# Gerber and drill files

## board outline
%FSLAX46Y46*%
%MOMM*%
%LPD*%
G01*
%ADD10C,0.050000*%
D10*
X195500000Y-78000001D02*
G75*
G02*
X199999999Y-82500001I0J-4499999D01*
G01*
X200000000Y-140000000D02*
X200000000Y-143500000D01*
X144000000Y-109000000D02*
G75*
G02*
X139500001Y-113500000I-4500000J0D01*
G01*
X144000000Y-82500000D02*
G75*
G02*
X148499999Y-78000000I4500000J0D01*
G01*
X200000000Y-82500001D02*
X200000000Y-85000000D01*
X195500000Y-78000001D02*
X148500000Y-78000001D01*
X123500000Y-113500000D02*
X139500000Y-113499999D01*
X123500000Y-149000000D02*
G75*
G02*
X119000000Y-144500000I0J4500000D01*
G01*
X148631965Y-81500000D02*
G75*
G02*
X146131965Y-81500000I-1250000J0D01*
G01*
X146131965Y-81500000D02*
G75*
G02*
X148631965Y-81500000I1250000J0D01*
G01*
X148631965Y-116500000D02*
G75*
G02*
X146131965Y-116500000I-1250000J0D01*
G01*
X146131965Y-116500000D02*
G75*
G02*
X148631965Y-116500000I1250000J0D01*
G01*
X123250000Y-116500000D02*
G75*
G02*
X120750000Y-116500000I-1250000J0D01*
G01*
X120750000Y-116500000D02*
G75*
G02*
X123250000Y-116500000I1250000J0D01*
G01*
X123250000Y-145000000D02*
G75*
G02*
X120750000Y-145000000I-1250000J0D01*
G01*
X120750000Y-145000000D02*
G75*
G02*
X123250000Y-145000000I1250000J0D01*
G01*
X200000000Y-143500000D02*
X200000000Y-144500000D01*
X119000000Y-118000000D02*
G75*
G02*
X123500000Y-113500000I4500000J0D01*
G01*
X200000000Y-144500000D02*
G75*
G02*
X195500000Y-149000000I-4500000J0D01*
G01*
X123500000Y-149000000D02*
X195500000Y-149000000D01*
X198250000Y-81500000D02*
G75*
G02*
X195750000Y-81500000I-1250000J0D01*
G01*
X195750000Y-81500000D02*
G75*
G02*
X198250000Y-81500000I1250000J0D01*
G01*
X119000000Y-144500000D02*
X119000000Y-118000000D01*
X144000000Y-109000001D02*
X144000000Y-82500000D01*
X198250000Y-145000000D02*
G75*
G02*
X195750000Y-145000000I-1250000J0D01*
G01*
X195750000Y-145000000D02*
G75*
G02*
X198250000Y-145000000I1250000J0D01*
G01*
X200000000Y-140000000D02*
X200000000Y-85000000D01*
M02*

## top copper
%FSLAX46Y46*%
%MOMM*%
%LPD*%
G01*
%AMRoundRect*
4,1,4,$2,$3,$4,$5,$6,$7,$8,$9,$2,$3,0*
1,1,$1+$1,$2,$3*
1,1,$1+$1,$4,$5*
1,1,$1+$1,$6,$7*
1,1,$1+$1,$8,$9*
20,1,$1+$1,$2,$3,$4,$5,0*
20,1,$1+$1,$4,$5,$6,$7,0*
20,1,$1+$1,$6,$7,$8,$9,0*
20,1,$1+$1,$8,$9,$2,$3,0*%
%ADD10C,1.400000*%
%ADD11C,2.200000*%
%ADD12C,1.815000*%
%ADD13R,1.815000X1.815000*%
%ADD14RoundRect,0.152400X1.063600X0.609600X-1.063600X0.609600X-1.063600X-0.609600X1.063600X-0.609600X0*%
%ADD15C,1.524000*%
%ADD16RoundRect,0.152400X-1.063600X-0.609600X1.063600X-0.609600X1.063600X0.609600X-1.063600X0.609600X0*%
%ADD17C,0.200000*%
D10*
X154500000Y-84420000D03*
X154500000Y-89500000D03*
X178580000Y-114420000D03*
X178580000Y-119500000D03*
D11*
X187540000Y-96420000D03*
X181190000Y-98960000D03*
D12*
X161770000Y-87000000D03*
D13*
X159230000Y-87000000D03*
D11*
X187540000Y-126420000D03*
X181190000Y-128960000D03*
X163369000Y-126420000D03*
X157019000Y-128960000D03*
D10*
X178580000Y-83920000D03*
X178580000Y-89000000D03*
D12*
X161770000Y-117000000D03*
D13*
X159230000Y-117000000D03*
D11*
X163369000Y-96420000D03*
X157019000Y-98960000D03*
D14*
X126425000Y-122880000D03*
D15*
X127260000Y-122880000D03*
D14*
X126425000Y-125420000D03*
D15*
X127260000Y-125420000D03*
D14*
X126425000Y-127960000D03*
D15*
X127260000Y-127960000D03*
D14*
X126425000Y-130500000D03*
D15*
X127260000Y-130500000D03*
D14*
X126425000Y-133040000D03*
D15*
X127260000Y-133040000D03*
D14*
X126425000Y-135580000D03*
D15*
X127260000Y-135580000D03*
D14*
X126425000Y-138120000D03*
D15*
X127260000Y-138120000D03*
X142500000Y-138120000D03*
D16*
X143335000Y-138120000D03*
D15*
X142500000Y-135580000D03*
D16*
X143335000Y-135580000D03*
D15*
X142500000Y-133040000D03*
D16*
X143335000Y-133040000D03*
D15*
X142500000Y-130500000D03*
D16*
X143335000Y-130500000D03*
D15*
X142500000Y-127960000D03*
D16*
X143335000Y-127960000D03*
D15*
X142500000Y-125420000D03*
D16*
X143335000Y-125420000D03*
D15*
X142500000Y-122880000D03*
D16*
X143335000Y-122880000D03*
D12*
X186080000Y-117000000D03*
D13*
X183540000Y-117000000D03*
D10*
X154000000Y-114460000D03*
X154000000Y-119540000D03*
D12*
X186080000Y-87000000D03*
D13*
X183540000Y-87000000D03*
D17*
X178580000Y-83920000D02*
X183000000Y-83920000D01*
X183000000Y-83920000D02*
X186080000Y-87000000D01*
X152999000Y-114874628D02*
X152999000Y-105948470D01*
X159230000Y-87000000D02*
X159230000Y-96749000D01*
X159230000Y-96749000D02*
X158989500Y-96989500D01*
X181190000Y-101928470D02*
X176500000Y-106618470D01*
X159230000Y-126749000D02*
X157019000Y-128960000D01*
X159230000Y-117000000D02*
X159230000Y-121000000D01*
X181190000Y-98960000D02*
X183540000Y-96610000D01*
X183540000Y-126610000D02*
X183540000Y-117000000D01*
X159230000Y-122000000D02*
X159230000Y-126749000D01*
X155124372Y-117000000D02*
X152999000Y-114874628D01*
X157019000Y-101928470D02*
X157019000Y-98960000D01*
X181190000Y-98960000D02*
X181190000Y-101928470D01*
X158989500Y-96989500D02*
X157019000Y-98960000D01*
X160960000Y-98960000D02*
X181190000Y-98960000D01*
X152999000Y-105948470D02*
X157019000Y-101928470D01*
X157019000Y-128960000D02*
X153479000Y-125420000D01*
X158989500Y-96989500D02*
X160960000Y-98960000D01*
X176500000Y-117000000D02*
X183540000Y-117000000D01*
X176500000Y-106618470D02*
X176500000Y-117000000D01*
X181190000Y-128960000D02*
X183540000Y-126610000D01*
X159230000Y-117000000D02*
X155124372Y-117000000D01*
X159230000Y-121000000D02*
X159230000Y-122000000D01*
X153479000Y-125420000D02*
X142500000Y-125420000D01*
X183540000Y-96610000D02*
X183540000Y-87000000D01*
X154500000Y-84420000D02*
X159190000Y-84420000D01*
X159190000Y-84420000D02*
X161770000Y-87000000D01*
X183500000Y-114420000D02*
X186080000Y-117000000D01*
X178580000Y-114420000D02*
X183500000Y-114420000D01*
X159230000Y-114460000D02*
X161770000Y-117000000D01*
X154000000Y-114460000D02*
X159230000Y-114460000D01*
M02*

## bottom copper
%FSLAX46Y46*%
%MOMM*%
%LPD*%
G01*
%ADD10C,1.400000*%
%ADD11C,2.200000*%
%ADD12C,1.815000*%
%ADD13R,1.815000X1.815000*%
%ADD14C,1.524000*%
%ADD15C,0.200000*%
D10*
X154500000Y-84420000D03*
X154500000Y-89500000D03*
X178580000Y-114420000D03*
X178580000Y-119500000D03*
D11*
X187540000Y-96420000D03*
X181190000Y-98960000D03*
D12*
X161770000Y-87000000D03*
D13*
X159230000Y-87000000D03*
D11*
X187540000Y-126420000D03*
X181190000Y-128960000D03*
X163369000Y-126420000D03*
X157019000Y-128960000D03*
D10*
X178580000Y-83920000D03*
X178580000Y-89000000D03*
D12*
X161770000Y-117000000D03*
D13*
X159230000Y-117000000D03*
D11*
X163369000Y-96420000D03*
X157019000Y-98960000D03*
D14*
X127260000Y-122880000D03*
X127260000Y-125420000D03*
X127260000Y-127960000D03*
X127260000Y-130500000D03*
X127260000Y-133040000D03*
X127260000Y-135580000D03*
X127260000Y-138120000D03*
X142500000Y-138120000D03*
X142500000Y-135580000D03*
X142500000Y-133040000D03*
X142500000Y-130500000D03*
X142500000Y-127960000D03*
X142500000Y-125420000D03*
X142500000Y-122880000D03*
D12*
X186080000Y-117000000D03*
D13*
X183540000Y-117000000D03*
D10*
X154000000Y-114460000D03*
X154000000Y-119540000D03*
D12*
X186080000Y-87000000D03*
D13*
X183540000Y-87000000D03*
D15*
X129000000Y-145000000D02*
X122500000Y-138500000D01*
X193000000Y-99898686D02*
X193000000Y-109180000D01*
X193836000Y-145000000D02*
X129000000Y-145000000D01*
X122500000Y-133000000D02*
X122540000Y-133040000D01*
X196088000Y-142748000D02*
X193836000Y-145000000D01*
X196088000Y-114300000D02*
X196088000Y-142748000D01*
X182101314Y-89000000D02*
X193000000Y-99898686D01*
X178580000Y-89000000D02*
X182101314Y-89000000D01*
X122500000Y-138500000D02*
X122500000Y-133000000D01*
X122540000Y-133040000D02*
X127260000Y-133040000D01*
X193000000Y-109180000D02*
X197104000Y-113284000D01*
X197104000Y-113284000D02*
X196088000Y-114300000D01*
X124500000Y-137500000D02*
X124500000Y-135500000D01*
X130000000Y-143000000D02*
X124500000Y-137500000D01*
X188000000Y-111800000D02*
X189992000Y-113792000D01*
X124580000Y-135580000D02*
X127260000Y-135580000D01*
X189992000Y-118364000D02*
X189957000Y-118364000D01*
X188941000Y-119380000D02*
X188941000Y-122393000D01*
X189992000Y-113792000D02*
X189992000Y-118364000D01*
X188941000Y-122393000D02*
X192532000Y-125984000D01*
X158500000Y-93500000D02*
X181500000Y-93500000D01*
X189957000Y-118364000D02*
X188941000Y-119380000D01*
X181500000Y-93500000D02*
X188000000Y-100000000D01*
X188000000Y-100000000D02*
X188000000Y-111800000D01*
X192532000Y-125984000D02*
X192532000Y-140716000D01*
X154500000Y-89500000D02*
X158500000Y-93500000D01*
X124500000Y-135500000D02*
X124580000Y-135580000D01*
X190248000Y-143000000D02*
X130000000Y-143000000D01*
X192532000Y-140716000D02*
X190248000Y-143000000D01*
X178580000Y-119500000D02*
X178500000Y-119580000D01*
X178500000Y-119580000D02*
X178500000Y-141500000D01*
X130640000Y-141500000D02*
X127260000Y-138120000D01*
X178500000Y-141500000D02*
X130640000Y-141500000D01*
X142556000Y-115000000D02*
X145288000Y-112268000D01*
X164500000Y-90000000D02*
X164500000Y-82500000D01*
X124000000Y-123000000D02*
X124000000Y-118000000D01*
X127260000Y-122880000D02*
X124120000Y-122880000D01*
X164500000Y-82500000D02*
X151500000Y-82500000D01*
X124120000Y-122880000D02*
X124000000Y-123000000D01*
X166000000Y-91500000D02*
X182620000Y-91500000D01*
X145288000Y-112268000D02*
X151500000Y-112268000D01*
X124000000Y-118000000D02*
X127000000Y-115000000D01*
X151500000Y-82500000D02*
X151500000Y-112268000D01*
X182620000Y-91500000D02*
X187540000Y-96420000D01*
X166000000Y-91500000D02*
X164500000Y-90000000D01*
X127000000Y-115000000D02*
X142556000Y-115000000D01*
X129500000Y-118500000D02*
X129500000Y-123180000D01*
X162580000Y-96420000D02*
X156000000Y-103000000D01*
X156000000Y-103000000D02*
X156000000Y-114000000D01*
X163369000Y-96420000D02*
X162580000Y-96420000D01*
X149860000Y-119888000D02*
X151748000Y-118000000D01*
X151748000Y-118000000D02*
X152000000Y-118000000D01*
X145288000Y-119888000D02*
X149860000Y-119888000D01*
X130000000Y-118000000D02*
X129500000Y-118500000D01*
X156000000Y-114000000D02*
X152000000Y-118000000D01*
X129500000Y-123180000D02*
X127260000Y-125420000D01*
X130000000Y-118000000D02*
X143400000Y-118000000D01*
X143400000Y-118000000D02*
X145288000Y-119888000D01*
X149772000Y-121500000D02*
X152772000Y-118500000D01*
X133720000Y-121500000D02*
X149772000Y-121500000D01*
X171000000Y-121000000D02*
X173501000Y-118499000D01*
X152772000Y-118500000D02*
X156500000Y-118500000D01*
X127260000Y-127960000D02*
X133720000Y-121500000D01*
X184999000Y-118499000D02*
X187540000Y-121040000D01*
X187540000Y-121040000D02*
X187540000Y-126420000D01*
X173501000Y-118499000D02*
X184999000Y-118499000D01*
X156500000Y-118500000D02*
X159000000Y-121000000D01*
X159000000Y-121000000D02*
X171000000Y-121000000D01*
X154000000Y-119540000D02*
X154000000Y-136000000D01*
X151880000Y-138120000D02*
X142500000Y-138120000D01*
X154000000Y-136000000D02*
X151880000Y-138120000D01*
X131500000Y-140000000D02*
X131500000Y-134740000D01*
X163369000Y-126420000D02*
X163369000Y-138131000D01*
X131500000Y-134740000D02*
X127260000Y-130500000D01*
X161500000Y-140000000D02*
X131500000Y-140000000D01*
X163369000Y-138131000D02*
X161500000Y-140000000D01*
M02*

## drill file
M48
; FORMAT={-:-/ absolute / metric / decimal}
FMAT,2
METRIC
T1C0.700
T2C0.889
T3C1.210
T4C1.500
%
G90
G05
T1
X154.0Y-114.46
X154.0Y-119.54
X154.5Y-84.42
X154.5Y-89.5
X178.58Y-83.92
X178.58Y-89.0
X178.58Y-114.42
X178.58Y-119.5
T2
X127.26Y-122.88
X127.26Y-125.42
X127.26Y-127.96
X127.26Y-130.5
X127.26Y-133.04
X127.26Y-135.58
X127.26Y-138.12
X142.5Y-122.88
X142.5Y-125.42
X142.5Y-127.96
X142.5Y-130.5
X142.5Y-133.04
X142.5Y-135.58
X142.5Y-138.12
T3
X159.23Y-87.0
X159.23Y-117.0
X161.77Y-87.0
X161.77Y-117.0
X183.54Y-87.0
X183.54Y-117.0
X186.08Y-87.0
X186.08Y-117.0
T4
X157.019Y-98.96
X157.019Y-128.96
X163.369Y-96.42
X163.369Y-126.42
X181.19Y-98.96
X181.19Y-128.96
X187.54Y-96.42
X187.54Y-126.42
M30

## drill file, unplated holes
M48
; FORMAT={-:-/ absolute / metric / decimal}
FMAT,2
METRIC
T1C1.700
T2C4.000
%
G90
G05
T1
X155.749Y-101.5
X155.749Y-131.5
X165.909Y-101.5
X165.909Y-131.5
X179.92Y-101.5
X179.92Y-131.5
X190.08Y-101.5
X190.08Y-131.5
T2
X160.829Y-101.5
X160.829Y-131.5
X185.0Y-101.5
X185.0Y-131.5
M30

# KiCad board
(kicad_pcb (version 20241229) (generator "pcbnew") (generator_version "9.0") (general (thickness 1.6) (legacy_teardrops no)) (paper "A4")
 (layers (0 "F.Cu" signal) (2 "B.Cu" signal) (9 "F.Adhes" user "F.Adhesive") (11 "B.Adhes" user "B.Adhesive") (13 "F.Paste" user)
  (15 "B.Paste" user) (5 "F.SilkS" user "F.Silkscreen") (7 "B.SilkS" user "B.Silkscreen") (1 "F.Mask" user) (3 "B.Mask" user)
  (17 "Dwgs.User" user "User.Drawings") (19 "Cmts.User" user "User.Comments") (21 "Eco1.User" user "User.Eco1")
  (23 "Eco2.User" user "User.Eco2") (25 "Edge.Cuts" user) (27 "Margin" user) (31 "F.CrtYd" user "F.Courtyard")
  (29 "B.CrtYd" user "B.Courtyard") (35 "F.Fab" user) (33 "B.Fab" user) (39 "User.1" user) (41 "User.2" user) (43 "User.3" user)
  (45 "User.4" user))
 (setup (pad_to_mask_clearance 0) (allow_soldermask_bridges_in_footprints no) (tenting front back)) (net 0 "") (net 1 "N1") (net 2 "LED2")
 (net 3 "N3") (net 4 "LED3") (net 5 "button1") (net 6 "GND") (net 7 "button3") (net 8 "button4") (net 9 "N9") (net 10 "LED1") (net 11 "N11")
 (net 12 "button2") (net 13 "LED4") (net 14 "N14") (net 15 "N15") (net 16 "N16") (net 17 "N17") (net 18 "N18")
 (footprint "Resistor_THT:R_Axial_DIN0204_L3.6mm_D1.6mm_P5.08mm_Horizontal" (layer "F.Cu") (at 154.5 84.42 -90)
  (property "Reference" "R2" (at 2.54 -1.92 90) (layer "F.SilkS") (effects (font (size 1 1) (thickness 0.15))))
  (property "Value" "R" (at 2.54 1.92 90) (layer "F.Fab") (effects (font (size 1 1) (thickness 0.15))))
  (pad "1" thru_hole circle (at 0 0 270) (size 1.4 1.4) (drill 0.7) (layers "*.Cu" "*.Mask") (remove_unused_layers no) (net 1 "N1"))
  (pad "2" thru_hole circle (at 5.08 0 270) (size 1.4 1.4) (drill 0.7) (layers "*.Cu" "*.Mask") (remove_unused_layers no) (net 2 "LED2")))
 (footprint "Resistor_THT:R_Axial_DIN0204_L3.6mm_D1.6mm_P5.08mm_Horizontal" (layer "F.Cu") (at 178.58 114.42 -90)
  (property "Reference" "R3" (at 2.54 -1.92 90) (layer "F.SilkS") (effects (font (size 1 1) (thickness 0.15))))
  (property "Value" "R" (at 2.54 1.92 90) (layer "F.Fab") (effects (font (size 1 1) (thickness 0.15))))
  (pad "1" thru_hole circle (at 0 0 270) (size 1.4 1.4) (drill 0.7) (layers "*.Cu" "*.Mask") (remove_unused_layers no) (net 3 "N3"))
  (pad "2" thru_hole circle (at 5.08 0 270) (size 1.4 1.4) (drill 0.7) (layers "*.Cu" "*.Mask") (remove_unused_layers no) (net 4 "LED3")))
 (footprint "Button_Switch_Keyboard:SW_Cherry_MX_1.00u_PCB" (layer "F.Cu") (at 187.54 96.42)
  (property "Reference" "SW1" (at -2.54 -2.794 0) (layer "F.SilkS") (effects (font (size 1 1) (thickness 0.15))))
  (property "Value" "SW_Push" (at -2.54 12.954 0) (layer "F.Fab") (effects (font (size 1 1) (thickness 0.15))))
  (pad "" np_thru_hole circle (at -7.62 5.08) (size 1.7 1.7) (drill 1.7) (layers "*.Cu" "*.Mask"))
  (pad "" np_thru_hole circle (at -2.54 5.08) (size 4 4) (drill 4) (layers "*.Cu" "*.Mask"))
  (pad "" np_thru_hole circle (at 2.54 5.08) (size 1.7 1.7) (drill 1.7) (layers "*.Cu" "*.Mask"))
  (pad "1" thru_hole circle (at 0 0) (size 2.2 2.2) (drill 1.5) (layers "*.Cu" "*.Mask") (remove_unused_layers no) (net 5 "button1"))
  (pad "2" thru_hole circle (at -6.35 2.54) (size 2.2 2.2) (drill 1.5) (layers "*.Cu" "*.Mask") (remove_unused_layers no) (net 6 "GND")))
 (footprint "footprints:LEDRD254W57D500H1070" (layer "F.Cu") (at 160.5 87)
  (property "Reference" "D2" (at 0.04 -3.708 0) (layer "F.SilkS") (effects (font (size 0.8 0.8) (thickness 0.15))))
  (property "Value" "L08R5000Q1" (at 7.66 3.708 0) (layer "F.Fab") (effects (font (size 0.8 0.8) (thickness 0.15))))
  (pad "A" thru_hole circle (at 1.27 0) (size 1.815 1.815) (drill 1.21) (layers "*.Cu" "*.Mask") (remove_unused_layers no) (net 1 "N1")
   (solder_mask_margin 0.102))
  (pad "C" thru_hole rect (at -1.27 0) (size 1.815 1.815) (drill 1.21) (layers "*.Cu" "*.Mask") (remove_unused_layers no) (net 6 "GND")
   (solder_mask_margin 0.102)))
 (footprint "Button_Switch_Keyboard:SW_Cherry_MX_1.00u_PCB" (layer "F.Cu") (at 187.54 126.42)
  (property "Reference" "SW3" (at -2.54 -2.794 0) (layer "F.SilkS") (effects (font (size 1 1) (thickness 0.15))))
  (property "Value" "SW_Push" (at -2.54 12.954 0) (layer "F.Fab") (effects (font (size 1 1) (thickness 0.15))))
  (pad "" np_thru_hole circle (at -7.62 5.08) (size 1.7 1.7) (drill 1.7) (layers "*.Cu" "*.Mask"))
  (pad "" np_thru_hole circle (at -2.54 5.08) (size 4 4) (drill 4) (layers "*.Cu" "*.Mask"))
  (pad "" np_thru_hole circle (at 2.54 5.08) (size 1.7 1.7) (drill 1.7) (layers "*.Cu" "*.Mask"))
  (pad "1" thru_hole circle (at 0 0) (size 2.2 2.2) (drill 1.5) (layers "*.Cu" "*.Mask") (remove_unused_layers no) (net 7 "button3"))
  (pad "2" thru_hole circle (at -6.35 2.54) (size 2.2 2.2) (drill 1.5) (layers "*.Cu" "*.Mask") (remove_unused_layers no) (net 6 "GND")))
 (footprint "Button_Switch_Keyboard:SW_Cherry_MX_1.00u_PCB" (layer "F.Cu") (at 163.369 126.42)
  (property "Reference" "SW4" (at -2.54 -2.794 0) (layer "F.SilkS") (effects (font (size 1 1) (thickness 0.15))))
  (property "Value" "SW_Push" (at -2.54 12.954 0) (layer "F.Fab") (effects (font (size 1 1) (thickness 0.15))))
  (pad "" np_thru_hole circle (at -7.62 5.08) (size 1.7 1.7) (drill 1.7) (layers "*.Cu" "*.Mask"))
  (pad "" np_thru_hole circle (at -2.54 5.08) (size 4 4) (drill 4) (layers "*.Cu" "*.Mask"))
  (pad "" np_thru_hole circle (at 2.54 5.08) (size 1.7 1.7) (drill 1.7) (layers "*.Cu" "*.Mask"))
  (pad "1" thru_hole circle (at 0 0) (size 2.2 2.2) (drill 1.5) (layers "*.Cu" "*.Mask") (remove_unused_layers no) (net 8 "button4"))
  (pad "2" thru_hole circle (at -6.35 2.54) (size 2.2 2.2) (drill 1.5) (layers "*.Cu" "*.Mask") (remove_unused_layers no) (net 6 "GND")))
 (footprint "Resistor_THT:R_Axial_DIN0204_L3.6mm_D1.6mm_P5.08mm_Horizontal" (layer "F.Cu") (at 178.58 83.92 -90)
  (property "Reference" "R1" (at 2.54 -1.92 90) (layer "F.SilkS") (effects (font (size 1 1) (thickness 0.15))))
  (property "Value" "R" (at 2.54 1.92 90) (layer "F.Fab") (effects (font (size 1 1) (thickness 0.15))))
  (pad "1" thru_hole circle (at 0 0 270) (size 1.4 1.4) (drill 0.7) (layers "*.Cu" "*.Mask") (remove_unused_layers no) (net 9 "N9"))
  (pad "2" thru_hole circle (at 5.08 0 270) (size 1.4 1.4) (drill 0.7) (layers "*.Cu" "*.Mask") (remove_unused_layers no) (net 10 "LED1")))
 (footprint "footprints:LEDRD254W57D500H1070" (layer "F.Cu") (at 160.5 117)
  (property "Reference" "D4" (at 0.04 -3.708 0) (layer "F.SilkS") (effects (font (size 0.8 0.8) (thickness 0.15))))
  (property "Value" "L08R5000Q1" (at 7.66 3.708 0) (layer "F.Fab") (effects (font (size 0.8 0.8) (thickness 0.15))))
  (pad "A" thru_hole circle (at 1.27 0) (size 1.815 1.815) (drill 1.21) (layers "*.Cu" "*.Mask") (remove_unused_layers no) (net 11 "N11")
   (solder_mask_margin 0.102))
  (pad "C" thru_hole rect (at -1.27 0) (size 1.815 1.815) (drill 1.21) (layers "*.Cu" "*.Mask") (remove_unused_layers no) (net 6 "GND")
   (solder_mask_margin 0.102)))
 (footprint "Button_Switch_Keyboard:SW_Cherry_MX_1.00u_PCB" (layer "F.Cu") (at 163.369 96.42)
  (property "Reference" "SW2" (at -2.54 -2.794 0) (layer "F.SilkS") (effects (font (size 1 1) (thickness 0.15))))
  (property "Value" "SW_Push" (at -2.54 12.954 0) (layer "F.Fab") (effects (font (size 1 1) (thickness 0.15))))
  (pad "" np_thru_hole circle (at -7.62 5.08) (size 1.7 1.7) (drill 1.7) (layers "*.Cu" "*.Mask"))
  (pad "" np_thru_hole circle (at -2.54 5.08) (size 4 4) (drill 4) (layers "*.Cu" "*.Mask"))
  (pad "" np_thru_hole circle (at 2.54 5.08) (size 1.7 1.7) (drill 1.7) (layers "*.Cu" "*.Mask"))
  (pad "1" thru_hole circle (at 0 0) (size 2.2 2.2) (drill 1.5) (layers "*.Cu" "*.Mask") (remove_unused_layers no) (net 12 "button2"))
  (pad "2" thru_hole circle (at -6.35 2.54) (size 2.2 2.2) (drill 1.5) (layers "*.Cu" "*.Mask") (remove_unused_layers no) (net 6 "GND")))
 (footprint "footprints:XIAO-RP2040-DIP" (layer "F.Cu") (at 134.88 130.5)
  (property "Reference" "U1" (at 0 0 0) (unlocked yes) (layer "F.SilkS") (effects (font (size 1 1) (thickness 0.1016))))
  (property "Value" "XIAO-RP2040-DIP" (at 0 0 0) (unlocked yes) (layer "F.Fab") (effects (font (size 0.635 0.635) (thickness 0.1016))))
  (pad "1" smd roundrect (at -8.455 -7.62 180) (size 2.432 1.524) (layers "F.Cu" "F.Mask") (roundrect_rratio 0.1) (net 5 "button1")
   (thermal_bridge_angle 45))
  (pad "1" thru_hole circle (at -7.62 -7.62 180) (size 1.524 1.524) (drill 0.889) (layers "*.Cu" "*.Mask") (remove_unused_layers no)
   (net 5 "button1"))
  (pad "2" smd roundrect (at -8.455 -5.08 180) (size 2.432 1.524) (layers "F.Cu" "F.Mask") (roundrect_rratio 0.1) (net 12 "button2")
   (thermal_bridge_angle 45))
  (pad "2" thru_hole circle (at -7.62 -5.08 180) (size 1.524 1.524) (drill 0.889) (layers "*.Cu" "*.Mask") (remove_unused_layers no)
   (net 12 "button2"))
  (pad "3" smd roundrect (at -8.455 -2.54 180) (size 2.432 1.524) (layers "F.Cu" "F.Mask") (roundrect_rratio 0.1) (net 7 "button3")
   (thermal_bridge_angle 45))
  (pad "3" thru_hole circle (at -7.62 -2.54 180) (size 1.524 1.524) (drill 0.889) (layers "*.Cu" "*.Mask") (remove_unused_layers no)
   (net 7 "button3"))
  (pad "4" smd roundrect (at -8.455 0 180) (size 2.432 1.524) (layers "F.Cu" "F.Mask") (roundrect_rratio 0.1) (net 8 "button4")
   (thermal_bridge_angle 45))
  (pad "4" thru_hole circle (at -7.62 0 180) (size 1.524 1.524) (drill 0.889) (layers "*.Cu" "*.Mask") (remove_unused_layers no)
   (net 8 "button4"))
  (pad "5" smd roundrect (at -8.455 2.54 180) (size 2.432 1.524) (layers "F.Cu" "F.Mask") (roundrect_rratio 0.1) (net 10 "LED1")
   (thermal_bridge_angle 45))
  (pad "5" thru_hole circle (at -7.62 2.54 180) (size 1.524 1.524) (drill 0.889) (layers "*.Cu" "*.Mask") (remove_unused_layers no)
   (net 10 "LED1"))
  (pad "6" smd roundrect (at -8.455 5.08 180) (size 2.432 1.524) (layers "F.Cu" "F.Mask") (roundrect_rratio 0.1) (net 2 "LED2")
   (thermal_bridge_angle 45))
  (pad "6" thru_hole circle (at -7.62 5.08 180) (size 1.524 1.524) (drill 0.889) (layers "*.Cu" "*.Mask") (remove_unused_layers no)
   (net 2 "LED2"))
  (pad "7" smd roundrect (at -8.455 7.62 180) (size 2.432 1.524) (layers "F.Cu" "F.Mask") (roundrect_rratio 0.1) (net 4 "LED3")
   (thermal_bridge_angle 45))
  (pad "7" thru_hole circle (at -7.62 7.62 180) (size 1.524 1.524) (drill 0.889) (layers "*.Cu" "*.Mask") (remove_unused_layers no)
   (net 4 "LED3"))
  (pad "8" thru_hole circle (at 7.62 7.62) (size 1.524 1.524) (drill 0.889) (layers "*.Cu" "*.Mask") (remove_unused_layers no)
   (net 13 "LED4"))
  (pad "8" smd roundrect (at 8.455 7.62) (size 2.432 1.524) (layers "F.Cu" "F.Mask") (roundrect_rratio 0.1) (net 13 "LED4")
   (thermal_bridge_angle 45))
  (pad "9" thru_hole circle (at 7.62 5.08) (size 1.524 1.524) (drill 0.889) (layers "*.Cu" "*.Mask") (remove_unused_layers no)
   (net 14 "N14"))
  (pad "9" smd roundrect (at 8.455 5.08) (size 2.432 1.524) (layers "F.Cu" "F.Mask") (roundrect_rratio 0.1) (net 14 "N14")
   (thermal_bridge_angle 45))
  (pad "10" thru_hole circle (at 7.62 2.54) (size 1.524 1.524) (drill 0.889) (layers "*.Cu" "*.Mask") (remove_unused_layers no)
   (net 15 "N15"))
  (pad "10" smd roundrect (at 8.455 2.54) (size 2.432 1.524) (layers "F.Cu" "F.Mask") (roundrect_rratio 0.1) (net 15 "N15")
   (thermal_bridge_angle 45))
  (pad "11" thru_hole circle (at 7.62 0) (size 1.524 1.524) (drill 0.889) (layers "*.Cu" "*.Mask") (remove_unused_layers no) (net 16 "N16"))
  (pad "11" smd roundrect (at 8.455 0) (size 2.432 1.524) (layers "F.Cu" "F.Mask") (roundrect_rratio 0.1) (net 16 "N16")
   (thermal_bridge_angle 45))
  (pad "12" thru_hole circle (at 7.62 -2.54) (size 1.524 1.524) (drill 0.889) (layers "*.Cu" "*.Mask") (remove_unused_layers no)
   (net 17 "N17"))
  (pad "12" smd roundrect (at 8.455 -2.54) (size 2.432 1.524) (layers "F.Cu" "F.Mask") (roundrect_rratio 0.1) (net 17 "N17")
   (thermal_bridge_angle 45))
  (pad "13" thru_hole circle (at 7.62 -5.08) (size 1.524 1.524) (drill 0.889) (layers "*.Cu" "*.Mask") (remove_unused_layers no)
   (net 6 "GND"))
  (pad "13" smd roundrect (at 8.455 -5.08) (size 2.432 1.524) (layers "F.Cu" "F.Mask") (roundrect_rratio 0.1) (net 6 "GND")
   (thermal_bridge_angle 45))
  (pad "14" thru_hole circle (at 7.62 -7.62) (size 1.524 1.524) (drill 0.889) (layers "*.Cu" "*.Mask") (remove_unused_layers no)
   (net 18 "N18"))
  (pad "14" smd roundrect (at 8.455 -7.62) (size 2.432 1.524) (layers "F.Cu" "F.Mask") (roundrect_rratio 0.1) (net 18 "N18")
   (thermal_bridge_angle 45)))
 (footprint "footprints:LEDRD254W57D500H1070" (layer "F.Cu") (at 184.81 117)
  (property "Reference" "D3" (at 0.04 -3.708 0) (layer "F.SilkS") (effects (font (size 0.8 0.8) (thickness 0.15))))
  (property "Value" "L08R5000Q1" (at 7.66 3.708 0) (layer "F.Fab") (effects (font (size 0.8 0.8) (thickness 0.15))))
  (pad "A" thru_hole circle (at 1.27 0) (size 1.815 1.815) (drill 1.21) (layers "*.Cu" "*.Mask") (remove_unused_layers no) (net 3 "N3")
   (solder_mask_margin 0.102))
  (pad "C" thru_hole rect (at -1.27 0) (size 1.815 1.815) (drill 1.21) (layers "*.Cu" "*.Mask") (remove_unused_layers no) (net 6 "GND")
   (solder_mask_margin 0.102)))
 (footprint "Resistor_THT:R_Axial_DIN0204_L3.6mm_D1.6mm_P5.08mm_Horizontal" (layer "F.Cu") (at 154 114.46 -90)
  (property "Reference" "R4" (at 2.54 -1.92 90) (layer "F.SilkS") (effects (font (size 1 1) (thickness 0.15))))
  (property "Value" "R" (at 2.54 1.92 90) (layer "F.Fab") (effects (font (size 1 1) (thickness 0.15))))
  (pad "1" thru_hole circle (at 0 0 270) (size 1.4 1.4) (drill 0.7) (layers "*.Cu" "*.Mask") (remove_unused_layers no) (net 11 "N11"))
  (pad "2" thru_hole circle (at 5.08 0 270) (size 1.4 1.4) (drill 0.7) (layers "*.Cu" "*.Mask") (remove_unused_layers no) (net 13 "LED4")))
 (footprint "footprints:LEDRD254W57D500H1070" (layer "F.Cu") (at 184.81 87)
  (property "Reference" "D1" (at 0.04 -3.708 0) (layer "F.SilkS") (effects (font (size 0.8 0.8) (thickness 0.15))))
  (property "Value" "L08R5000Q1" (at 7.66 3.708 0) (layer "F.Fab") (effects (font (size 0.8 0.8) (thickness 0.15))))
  (pad "A" thru_hole circle (at 1.27 0) (size 1.815 1.815) (drill 1.21) (layers "*.Cu" "*.Mask") (remove_unused_layers no) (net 9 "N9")
   (solder_mask_margin 0.102))
  (pad "C" thru_hole rect (at -1.27 0) (size 1.815 1.815) (drill 1.21) (layers "*.Cu" "*.Mask") (remove_unused_layers no) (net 6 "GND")
   (solder_mask_margin 0.102)))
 (gr_arc (start 195.5 78.000001) (mid 198.681981 79.31802) (end 200 82.500001) (stroke (width 0.05) (type default)) (layer "Edge.Cuts"))
 (gr_line (start 200 140) (end 200 143.5) (stroke (width 0.05) (type default)) (layer "Edge.Cuts"))
 (gr_arc (start 144 109) (mid 142.681982 112.181986) (end 139.500001 113.499999) (stroke (width 0.05) (type default)) (layer "Edge.Cuts"))
 (gr_arc (start 144 82.5) (mid 145.31802 79.318026) (end 148.499999 78.000001) (stroke (width 0.05) (type default)) (layer "Edge.Cuts"))
 (gr_line (start 200 82.500001) (end 200 85) (stroke (width 0.05) (type default)) (layer "Edge.Cuts"))
 (gr_line (start 195.5 78.000001) (end 148.5 78.000001) (stroke (width 0.05) (type default)) (layer "Edge.Cuts"))
 (gr_line (start 123.5 113.5) (end 139.5 113.499999) (stroke (width 0.05) (type default)) (layer "Edge.Cuts"))
 (gr_arc (start 123.5 149) (mid 120.318019 147.681981) (end 119 144.5) (stroke (width 0.05) (type default)) (layer "Edge.Cuts"))
 (gr_circle (center 147.381965 81.5) (end 148.631965 81.5) (stroke (width 0.05) (type solid)) (fill no) (layer "Edge.Cuts"))
 (gr_circle (center 147.381965 116.5) (end 148.631965 116.5) (stroke (width 0.05) (type solid)) (fill no) (layer "Edge.Cuts"))
 (gr_circle (center 122 116.5) (end 123.25 116.5) (stroke (width 0.05) (type solid)) (fill no) (layer "Edge.Cuts"))
 (gr_circle (center 122 145) (end 123.25 145) (stroke (width 0.05) (type solid)) (fill no) (layer "Edge.Cuts"))
 (gr_line (start 200 143.5) (end 200 144.5) (stroke (width 0.05) (type default)) (layer "Edge.Cuts"))
 (gr_arc (start 119 118) (mid 120.31802 114.81802) (end 123.5 113.5) (stroke (width 0.05) (type default)) (layer "Edge.Cuts"))
 (gr_arc (start 200 144.5) (mid 198.681981 147.681981) (end 195.5 149) (stroke (width 0.05) (type default)) (layer "Edge.Cuts"))
 (gr_line (start 123.5 149) (end 195.5 149) (stroke (width 0.05) (type default)) (layer "Edge.Cuts"))
 (gr_circle (center 197 81.5) (end 198.25 81.5) (stroke (width 0.05) (type solid)) (fill no) (layer "Edge.Cuts"))
 (gr_line (start 119 144.5) (end 119 118) (stroke (width 0.05) (type default)) (layer "Edge.Cuts"))
 (gr_line (start 144 109.000001) (end 144 82.5) (stroke (width 0.05) (type default)) (layer "Edge.Cuts"))
 (gr_circle (center 197 145) (end 198.25 145) (stroke (width 0.05) (type solid)) (fill no) (layer "Edge.Cuts"))
 (gr_line (start 200 140) (end 200 85) (stroke (width 0.05) (type solid)) (layer "Edge.Cuts"))
 (segment (start 178.58 83.92) (end 183 83.92) (width 0.2) (layer "F.Cu") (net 9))
 (segment (start 183 83.92) (end 186.08 87) (width 0.2) (layer "F.Cu") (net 9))
 (segment (start 152.999 114.874628) (end 152.999 105.94847) (width 0.2) (layer "F.Cu") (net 6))
 (segment (start 159.23 87) (end 159.23 96.749) (width 0.2) (layer "F.Cu") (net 6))
 (segment (start 159.23 96.749) (end 158.9895 96.9895) (width 0.2) (layer "F.Cu") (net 6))
 (segment (start 181.19 101.92847) (end 176.5 106.61847) (width 0.2) (layer "F.Cu") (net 6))
 (segment (start 159.23 126.749) (end 157.019 128.96) (width 0.2) (layer "F.Cu") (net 6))
 (segment (start 159.23 117) (end 159.23 121) (width 0.2) (layer "F.Cu") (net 6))
 (segment (start 181.19 98.96) (end 183.54 96.61) (width 0.2) (layer "F.Cu") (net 6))
 (segment (start 183.54 126.61) (end 183.54 117) (width 0.2) (layer "F.Cu") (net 6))
 (segment (start 159.23 122) (end 159.23 126.749) (width 0.2) (layer "F.Cu") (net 6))
 (segment (start 155.124372 117) (end 152.999 114.874628) (width 0.2) (layer "F.Cu") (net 6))
 (segment (start 157.019 101.92847) (end 157.019 98.96) (width 0.2) (layer "F.Cu") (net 6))
 (segment (start 181.19 98.96) (end 181.19 101.92847) (width 0.2) (layer "F.Cu") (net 6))
 (segment (start 158.9895 96.9895) (end 157.019 98.96) (width 0.2) (layer "F.Cu") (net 6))
 (segment (start 160.96 98.96) (end 181.19 98.96) (width 0.2) (layer "F.Cu") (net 6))
 (segment (start 152.999 105.94847) (end 157.019 101.92847) (width 0.2) (layer "F.Cu") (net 6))
 (segment (start 157.019 128.96) (end 153.479 125.42) (width 0.2) (layer "F.Cu") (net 6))
 (segment (start 158.9895 96.9895) (end 160.96 98.96) (width 0.2) (layer "F.Cu") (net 6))
 (segment (start 176.5 117) (end 183.54 117) (width 0.2) (layer "F.Cu") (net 6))
 (segment (start 176.5 106.61847) (end 176.5 117) (width 0.2) (layer "F.Cu") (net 6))
 (segment (start 181.19 128.96) (end 183.54 126.61) (width 0.2) (layer "F.Cu") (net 6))
 (segment (start 159.23 117) (end 155.124372 117) (width 0.2) (layer "F.Cu") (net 6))
 (segment (start 159.23 121) (end 159.23 122) (width 0.2) (layer "F.Cu") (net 6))
 (segment (start 153.479 125.42) (end 142.5 125.42) (width 0.2) (layer "F.Cu") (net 6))
 (segment (start 183.54 96.61) (end 183.54 87) (width 0.2) (layer "F.Cu") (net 6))
 (segment (start 154.5 84.42) (end 159.19 84.42) (width 0.2) (layer "F.Cu") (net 1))
 (segment (start 159.19 84.42) (end 161.77 87) (width 0.2) (layer "F.Cu") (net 1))
 (segment (start 183.5 114.42) (end 186.08 117) (width 0.2) (layer "F.Cu") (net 3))
 (segment (start 178.58 114.42) (end 183.5 114.42) (width 0.2) (layer "F.Cu") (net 3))
 (segment (start 129 145) (end 122.5 138.5) (width 0.2) (layer "B.Cu") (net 10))
 (segment (start 193 99.898686) (end 193 109.18) (width 0.2) (layer "B.Cu") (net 10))
 (segment (start 193.836 145) (end 129 145) (width 0.2) (layer "B.Cu") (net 10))
 (segment (start 122.5 133) (end 122.54 133.04) (width 0.2) (layer "B.Cu") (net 10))
 (segment (start 196.088 142.748) (end 193.836 145) (width 0.2) (layer "B.Cu") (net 10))
 (segment (start 196.088 114.3) (end 196.088 142.748) (width 0.2) (layer "B.Cu") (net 10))
 (segment (start 182.101314 89) (end 193 99.898686) (width 0.2) (layer "B.Cu") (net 10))
 (segment (start 178.58 89) (end 182.101314 89) (width 0.2) (layer "B.Cu") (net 10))
 (segment (start 122.5 138.5) (end 122.5 133) (width 0.2) (layer "B.Cu") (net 10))
 (segment (start 122.54 133.04) (end 127.26 133.04) (width 0.2) (layer "B.Cu") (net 10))
 (segment (start 193 109.18) (end 197.104 113.284) (width 0.2) (layer "B.Cu") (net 10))
 (segment (start 197.104 113.284) (end 196.088 114.3) (width 0.2) (layer "B.Cu") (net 10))
 (segment (start 124.5 137.5) (end 124.5 135.5) (width 0.2) (layer "B.Cu") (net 2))
 (segment (start 130 143) (end 124.5 137.5) (width 0.2) (layer "B.Cu") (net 2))
 (segment (start 188 111.8) (end 189.992 113.792) (width 0.2) (layer "B.Cu") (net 2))
 (segment (start 124.58 135.58) (end 127.26 135.58) (width 0.2) (layer "B.Cu") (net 2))
 (segment (start 189.992 118.364) (end 189.957 118.364) (width 0.2) (layer "B.Cu") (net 2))
 (segment (start 188.941 119.38) (end 188.941 122.393) (width 0.2) (layer "B.Cu") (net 2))
 (segment (start 189.992 113.792) (end 189.992 118.364) (width 0.2) (layer "B.Cu") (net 2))
 (segment (start 188.941 122.393) (end 192.532 125.984) (width 0.2) (layer "B.Cu") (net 2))
 (segment (start 158.5 93.5) (end 181.5 93.5) (width 0.2) (layer "B.Cu") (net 2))
 (segment (start 189.957 118.364) (end 188.941 119.38) (width 0.2) (layer "B.Cu") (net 2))
 (segment (start 181.5 93.5) (end 188 100) (width 0.2) (layer "B.Cu") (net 2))
 (segment (start 188 100) (end 188 111.8) (width 0.2) (layer "B.Cu") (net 2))
 (segment (start 192.532 125.984) (end 192.532 140.716) (width 0.2) (layer "B.Cu") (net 2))
 (segment (start 154.5 89.5) (end 158.5 93.5) (width 0.2) (layer "B.Cu") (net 2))
 (segment (start 124.5 135.5) (end 124.58 135.58) (width 0.2) (layer "B.Cu") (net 2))
 (segment (start 190.248 143) (end 130 143) (width 0.2) (layer "B.Cu") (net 2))
 (segment (start 192.532 140.716) (end 190.248 143) (width 0.2) (layer "B.Cu") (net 2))
 (segment (start 178.58 119.5) (end 178.5 119.58) (width 0.2) (layer "B.Cu") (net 4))
 (segment (start 178.5 119.58) (end 178.5 141.5) (width 0.2) (layer "B.Cu") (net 4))
 (segment (start 130.64 141.5) (end 127.26 138.12) (width 0.2) (layer "B.Cu") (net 4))
 (segment (start 178.5 141.5) (end 130.64 141.5) (width 0.2) (layer "B.Cu") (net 4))
 (segment (start 142.556 115) (end 145.288 112.268) (width 0.2) (layer "B.Cu") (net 5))
 (segment (start 164.5 90) (end 164.5 82.5) (width 0.2) (layer "B.Cu") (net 5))
 (segment (start 124 123) (end 124 118) (width 0.2) (layer "B.Cu") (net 5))
 (segment (start 127.26 122.88) (end 124.12 122.88) (width 0.2) (layer "B.Cu") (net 5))
 (segment (start 164.5 82.5) (end 151.5 82.5) (width 0.2) (layer "B.Cu") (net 5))
 (segment (start 124.12 122.88) (end 124 123) (width 0.2) (layer "B.Cu") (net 5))
 (segment (start 166 91.5) (end 182.62 91.5) (width 0.2) (layer "B.Cu") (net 5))
 (segment (start 145.288 112.268) (end 151.5 112.268) (width 0.2) (layer "B.Cu") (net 5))
 (segment (start 124 118) (end 127 115) (width 0.2) (layer "B.Cu") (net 5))
 (segment (start 151.5 82.5) (end 151.5 112.268) (width 0.2) (layer "B.Cu") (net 5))
 (segment (start 182.62 91.5) (end 187.54 96.42) (width 0.2) (layer "B.Cu") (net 5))
 (segment (start 166 91.5) (end 164.5 90) (width 0.2) (layer "B.Cu") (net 5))
 (segment (start 127 115) (end 142.556 115) (width 0.2) (layer "B.Cu") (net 5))
 (segment (start 129.5 118.5) (end 129.5 123.18) (width 0.2) (layer "B.Cu") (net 12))
 (segment (start 162.58 96.42) (end 156 103) (width 0.2) (layer "B.Cu") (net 12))
 (segment (start 156 103) (end 156 114) (width 0.2) (layer "B.Cu") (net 12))
 (segment (start 163.369 96.42) (end 162.58 96.42) (width 0.2) (layer "B.Cu") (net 12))
 (segment (start 149.86 119.888) (end 151.748 118) (width 0.2) (layer "B.Cu") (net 12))
 (segment (start 151.748 118) (end 152 118) (width 0.2) (layer "B.Cu") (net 12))
 (segment (start 145.288 119.888) (end 149.86 119.888) (width 0.2) (layer "B.Cu") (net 12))
 (segment (start 130 118) (end 129.5 118.5) (width 0.2) (layer "B.Cu") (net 12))
 (segment (start 156 114) (end 152 118) (width 0.2) (layer "B.Cu") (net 12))
 (segment (start 129.5 123.18) (end 127.26 125.42) (width 0.2) (layer "B.Cu") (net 12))
 (segment (start 130 118) (end 143.4 118) (width 0.2) (layer "B.Cu") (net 12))
 (segment (start 143.4 118) (end 145.288 119.888) (width 0.2) (layer "B.Cu") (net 12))
 (segment (start 149.772 121.5) (end 152.772 118.5) (width 0.2) (layer "B.Cu") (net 7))
 (segment (start 133.72 121.5) (end 149.772 121.5) (width 0.2) (layer "B.Cu") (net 7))
 (segment (start 171 121) (end 173.501 118.499) (width 0.2) (layer "B.Cu") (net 7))
 (segment (start 152.772 118.5) (end 156.5 118.5) (width 0.2) (layer "B.Cu") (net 7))
 (segment (start 127.26 127.96) (end 133.72 121.5) (width 0.2) (layer "B.Cu") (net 7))
 (segment (start 184.999 118.499) (end 187.54 121.04) (width 0.2) (layer "B.Cu") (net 7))
 (segment (start 187.54 121.04) (end 187.54 126.42) (width 0.2) (layer "B.Cu") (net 7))
 (segment (start 173.501 118.499) (end 184.999 118.499) (width 0.2) (layer "B.Cu") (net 7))
 (segment (start 156.5 118.5) (end 159 121) (width 0.2) (layer "B.Cu") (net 7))
 (segment (start 159 121) (end 171 121) (width 0.2) (layer "B.Cu") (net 7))
 (segment (start 159.23 114.46) (end 161.77 117) (width 0.2) (layer "F.Cu") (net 11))
 (segment (start 154 114.46) (end 159.23 114.46) (width 0.2) (layer "F.Cu") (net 11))
 (segment (start 154 119.54) (end 154 136) (width 0.2) (layer "B.Cu") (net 13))
 (segment (start 151.88 138.12) (end 142.5 138.12) (width 0.2) (layer "B.Cu") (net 13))
 (segment (start 154 136) (end 151.88 138.12) (width 0.2) (layer "B.Cu") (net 13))
 (segment (start 131.5 140) (end 131.5 134.74) (width 0.2) (layer "B.Cu") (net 8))
 (segment (start 163.369 126.42) (end 163.369 138.131) (width 0.2) (layer "B.Cu") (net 8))
 (segment (start 131.5 134.74) (end 127.26 130.5) (width 0.2) (layer "B.Cu") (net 8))
 (segment (start 161.5 140) (end 131.5 140) (width 0.2) (layer "B.Cu") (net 8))
 (segment (start 163.369 138.131) (end 161.5 140) (width 0.2) (layer "B.Cu") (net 8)))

